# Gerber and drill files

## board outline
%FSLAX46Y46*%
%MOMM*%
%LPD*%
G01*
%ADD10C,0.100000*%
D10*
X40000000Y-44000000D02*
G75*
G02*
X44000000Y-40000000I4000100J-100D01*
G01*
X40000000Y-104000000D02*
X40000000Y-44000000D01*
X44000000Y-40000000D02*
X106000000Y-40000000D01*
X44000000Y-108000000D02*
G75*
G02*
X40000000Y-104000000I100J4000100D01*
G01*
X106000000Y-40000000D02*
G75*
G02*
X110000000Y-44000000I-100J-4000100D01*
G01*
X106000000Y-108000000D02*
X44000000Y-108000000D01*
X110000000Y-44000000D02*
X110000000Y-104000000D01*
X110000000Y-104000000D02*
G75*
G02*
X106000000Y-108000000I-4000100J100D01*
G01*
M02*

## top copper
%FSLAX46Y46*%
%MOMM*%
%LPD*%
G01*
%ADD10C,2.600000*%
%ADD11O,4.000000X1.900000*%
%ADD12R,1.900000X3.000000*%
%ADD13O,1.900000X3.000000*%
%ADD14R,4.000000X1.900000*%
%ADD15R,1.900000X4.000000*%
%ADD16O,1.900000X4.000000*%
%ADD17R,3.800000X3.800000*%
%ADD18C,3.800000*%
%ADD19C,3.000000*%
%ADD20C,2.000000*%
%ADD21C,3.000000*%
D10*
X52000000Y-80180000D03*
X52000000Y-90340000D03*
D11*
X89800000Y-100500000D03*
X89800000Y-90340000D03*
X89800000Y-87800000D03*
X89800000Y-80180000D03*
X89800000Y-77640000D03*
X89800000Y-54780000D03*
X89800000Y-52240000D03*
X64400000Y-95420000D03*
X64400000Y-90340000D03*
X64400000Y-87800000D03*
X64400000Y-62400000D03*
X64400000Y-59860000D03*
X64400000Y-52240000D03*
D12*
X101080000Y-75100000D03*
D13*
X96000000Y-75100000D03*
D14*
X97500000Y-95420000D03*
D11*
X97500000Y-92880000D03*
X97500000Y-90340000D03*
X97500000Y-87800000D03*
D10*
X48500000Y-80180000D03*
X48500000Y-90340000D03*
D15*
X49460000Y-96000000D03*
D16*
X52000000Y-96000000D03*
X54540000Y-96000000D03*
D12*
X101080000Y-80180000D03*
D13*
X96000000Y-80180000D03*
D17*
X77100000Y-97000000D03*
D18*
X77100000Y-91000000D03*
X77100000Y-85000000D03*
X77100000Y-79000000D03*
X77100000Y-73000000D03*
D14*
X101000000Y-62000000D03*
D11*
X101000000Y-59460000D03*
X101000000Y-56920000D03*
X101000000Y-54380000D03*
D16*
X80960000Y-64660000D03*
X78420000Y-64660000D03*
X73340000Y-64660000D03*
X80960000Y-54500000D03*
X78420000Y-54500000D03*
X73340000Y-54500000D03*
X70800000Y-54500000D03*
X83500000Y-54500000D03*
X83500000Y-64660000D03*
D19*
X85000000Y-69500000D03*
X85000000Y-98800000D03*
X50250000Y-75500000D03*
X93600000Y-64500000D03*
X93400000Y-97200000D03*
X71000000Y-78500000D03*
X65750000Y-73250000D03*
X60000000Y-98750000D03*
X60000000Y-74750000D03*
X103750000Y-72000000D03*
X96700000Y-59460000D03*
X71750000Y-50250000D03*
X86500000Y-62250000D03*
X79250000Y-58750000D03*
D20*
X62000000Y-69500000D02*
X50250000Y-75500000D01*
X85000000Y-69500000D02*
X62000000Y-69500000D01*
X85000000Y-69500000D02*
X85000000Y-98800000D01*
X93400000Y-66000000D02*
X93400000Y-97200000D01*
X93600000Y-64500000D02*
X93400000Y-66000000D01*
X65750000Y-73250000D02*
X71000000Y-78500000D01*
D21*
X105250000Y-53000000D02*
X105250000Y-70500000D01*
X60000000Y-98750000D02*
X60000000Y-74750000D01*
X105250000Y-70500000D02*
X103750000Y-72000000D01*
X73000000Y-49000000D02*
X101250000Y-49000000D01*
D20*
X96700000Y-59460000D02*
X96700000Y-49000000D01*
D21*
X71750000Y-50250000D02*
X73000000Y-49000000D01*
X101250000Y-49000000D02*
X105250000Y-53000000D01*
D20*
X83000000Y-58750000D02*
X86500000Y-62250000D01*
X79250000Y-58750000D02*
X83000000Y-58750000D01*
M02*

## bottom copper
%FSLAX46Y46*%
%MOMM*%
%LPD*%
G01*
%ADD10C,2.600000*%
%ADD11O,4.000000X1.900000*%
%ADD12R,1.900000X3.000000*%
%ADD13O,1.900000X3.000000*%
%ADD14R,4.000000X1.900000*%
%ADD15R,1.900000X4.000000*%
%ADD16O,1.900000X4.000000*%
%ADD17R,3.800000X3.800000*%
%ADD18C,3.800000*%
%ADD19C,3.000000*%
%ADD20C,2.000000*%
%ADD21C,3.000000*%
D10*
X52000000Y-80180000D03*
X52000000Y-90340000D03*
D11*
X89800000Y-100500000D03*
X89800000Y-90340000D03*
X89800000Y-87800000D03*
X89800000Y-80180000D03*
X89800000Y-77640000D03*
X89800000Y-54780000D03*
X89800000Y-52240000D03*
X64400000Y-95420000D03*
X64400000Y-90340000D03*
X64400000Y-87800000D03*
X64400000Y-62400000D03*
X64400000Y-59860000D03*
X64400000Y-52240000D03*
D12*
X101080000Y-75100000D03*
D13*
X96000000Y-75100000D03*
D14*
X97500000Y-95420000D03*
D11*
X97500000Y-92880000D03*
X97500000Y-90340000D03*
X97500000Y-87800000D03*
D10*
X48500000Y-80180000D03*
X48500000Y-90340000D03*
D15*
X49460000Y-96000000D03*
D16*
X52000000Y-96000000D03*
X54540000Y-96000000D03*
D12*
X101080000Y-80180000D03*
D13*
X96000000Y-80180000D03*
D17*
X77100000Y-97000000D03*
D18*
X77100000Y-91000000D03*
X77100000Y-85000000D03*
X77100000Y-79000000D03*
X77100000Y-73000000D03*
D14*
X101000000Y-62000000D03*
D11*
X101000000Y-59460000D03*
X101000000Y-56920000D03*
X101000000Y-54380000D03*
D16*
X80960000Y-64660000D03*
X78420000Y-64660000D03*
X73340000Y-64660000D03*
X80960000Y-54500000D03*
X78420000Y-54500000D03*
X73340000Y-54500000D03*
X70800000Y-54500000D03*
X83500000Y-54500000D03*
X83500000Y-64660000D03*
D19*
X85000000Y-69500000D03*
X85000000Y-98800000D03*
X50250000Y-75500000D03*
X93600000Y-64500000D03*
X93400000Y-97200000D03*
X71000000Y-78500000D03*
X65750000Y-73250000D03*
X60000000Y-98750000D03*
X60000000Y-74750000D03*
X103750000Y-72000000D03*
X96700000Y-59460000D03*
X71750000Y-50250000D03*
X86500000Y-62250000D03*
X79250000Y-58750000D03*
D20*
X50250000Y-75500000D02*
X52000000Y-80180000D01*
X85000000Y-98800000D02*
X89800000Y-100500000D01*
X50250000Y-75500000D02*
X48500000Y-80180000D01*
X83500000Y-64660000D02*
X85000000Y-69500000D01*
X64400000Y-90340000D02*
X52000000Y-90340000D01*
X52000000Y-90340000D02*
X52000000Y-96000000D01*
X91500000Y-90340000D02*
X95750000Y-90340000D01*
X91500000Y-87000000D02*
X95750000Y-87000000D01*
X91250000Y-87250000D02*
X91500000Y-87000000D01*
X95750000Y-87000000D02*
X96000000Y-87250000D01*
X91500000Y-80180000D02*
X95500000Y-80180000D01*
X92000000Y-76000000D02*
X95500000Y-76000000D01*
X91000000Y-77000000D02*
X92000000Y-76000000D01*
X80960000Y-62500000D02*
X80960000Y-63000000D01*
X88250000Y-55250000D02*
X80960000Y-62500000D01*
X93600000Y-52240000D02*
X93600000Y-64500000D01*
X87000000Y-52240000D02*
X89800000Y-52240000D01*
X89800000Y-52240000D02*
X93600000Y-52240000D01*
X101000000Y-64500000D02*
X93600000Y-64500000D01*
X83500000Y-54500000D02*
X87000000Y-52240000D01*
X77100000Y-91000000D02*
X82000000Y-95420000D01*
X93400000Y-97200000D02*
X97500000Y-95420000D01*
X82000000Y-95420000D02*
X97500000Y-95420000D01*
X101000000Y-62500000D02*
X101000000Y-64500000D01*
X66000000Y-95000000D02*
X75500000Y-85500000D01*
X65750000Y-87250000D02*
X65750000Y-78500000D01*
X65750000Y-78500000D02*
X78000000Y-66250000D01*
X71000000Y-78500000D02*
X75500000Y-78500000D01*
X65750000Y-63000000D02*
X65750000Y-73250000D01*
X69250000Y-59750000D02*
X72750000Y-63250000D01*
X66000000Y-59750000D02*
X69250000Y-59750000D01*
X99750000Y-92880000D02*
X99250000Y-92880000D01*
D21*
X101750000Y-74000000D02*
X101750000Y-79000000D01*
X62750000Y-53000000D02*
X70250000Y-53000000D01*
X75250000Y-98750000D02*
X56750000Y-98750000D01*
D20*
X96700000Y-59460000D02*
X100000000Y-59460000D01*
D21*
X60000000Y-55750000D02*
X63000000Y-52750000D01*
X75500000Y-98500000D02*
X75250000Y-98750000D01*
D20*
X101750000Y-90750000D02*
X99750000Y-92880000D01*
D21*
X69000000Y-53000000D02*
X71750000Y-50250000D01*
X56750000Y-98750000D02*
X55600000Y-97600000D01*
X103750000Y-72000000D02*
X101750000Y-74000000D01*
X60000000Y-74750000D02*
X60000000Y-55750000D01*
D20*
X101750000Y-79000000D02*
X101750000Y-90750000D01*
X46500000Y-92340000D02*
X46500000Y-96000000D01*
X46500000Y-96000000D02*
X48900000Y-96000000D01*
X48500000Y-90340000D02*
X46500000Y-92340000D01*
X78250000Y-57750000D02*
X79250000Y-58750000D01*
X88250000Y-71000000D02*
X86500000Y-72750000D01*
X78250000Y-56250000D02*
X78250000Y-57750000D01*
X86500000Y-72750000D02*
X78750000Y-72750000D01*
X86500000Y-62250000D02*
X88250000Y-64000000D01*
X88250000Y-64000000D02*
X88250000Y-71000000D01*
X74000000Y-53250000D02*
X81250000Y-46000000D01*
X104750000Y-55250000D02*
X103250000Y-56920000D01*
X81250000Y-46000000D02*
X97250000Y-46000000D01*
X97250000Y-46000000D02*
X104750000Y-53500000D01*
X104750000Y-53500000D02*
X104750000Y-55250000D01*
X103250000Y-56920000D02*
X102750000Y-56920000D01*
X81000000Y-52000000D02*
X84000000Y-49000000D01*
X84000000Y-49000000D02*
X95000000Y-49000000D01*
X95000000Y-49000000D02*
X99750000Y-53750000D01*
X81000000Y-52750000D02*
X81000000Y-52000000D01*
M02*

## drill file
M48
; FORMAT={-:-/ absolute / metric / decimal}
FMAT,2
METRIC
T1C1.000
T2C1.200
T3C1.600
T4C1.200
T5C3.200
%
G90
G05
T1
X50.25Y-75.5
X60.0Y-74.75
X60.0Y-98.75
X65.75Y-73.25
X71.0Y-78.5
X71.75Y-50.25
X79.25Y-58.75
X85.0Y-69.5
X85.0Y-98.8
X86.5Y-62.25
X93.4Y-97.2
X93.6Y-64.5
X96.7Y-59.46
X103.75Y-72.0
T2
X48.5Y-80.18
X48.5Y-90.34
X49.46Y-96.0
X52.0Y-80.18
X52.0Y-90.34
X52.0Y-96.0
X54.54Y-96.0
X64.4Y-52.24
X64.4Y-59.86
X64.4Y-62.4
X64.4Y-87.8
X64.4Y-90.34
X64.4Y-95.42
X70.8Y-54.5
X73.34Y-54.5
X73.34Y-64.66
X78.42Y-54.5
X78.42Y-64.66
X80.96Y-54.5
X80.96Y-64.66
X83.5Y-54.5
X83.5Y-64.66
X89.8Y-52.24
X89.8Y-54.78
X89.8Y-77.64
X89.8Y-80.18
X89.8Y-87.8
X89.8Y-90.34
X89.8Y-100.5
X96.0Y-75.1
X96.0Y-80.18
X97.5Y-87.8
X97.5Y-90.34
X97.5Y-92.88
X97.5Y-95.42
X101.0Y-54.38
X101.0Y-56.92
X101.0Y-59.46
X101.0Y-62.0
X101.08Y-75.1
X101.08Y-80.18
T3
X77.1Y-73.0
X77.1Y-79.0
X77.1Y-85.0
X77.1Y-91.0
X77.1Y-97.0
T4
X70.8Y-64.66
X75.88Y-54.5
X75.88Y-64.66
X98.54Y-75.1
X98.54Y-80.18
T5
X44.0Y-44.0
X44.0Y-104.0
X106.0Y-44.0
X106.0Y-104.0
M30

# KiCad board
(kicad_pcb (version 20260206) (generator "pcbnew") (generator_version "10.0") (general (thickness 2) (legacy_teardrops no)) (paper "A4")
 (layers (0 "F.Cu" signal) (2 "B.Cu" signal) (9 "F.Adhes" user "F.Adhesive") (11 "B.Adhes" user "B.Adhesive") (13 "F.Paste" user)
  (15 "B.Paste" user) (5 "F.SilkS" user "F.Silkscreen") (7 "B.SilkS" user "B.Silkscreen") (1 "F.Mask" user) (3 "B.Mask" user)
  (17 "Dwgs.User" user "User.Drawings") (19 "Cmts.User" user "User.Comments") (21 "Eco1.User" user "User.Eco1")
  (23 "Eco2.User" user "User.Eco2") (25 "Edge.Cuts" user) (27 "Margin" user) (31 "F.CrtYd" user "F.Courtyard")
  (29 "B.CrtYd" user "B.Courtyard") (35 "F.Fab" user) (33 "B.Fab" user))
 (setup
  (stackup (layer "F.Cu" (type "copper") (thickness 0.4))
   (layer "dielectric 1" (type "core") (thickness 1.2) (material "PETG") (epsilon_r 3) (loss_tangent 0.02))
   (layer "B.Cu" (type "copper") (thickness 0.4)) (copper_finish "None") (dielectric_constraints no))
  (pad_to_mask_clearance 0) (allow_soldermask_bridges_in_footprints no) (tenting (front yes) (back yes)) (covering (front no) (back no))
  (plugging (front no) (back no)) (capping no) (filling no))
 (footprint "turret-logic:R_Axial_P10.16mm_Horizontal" (layer "F.Cu") (at 52 80.18 -90)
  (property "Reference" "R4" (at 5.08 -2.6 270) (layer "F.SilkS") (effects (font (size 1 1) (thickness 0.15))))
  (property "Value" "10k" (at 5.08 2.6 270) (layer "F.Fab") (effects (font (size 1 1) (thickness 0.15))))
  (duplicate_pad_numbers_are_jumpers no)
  (pad "1" thru_hole circle (at 0 0 270) (size 2.6 2.6) (drill 1.2) (layers "*.Cu" "*.Mask") (remove_unused_layers no) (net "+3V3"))
  (pad "2" thru_hole circle (at 10.16 0 270) (size 2.6 2.6) (drill 1.2) (layers "*.Cu" "*.Mask") (remove_unused_layers no) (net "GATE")))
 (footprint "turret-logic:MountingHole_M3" (layer "F.Cu") (at 106 44)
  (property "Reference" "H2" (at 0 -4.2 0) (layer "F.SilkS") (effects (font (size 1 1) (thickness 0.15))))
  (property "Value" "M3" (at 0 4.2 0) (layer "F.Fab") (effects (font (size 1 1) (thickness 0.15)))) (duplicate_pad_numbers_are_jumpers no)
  (pad "" np_thru_hole circle (at 0 0) (size 3.2 3.2) (drill 3.2) (layers "*.Cu" "*.Mask")))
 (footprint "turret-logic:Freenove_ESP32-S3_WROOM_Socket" (layer "F.Cu") (at 89.8 100.5 90)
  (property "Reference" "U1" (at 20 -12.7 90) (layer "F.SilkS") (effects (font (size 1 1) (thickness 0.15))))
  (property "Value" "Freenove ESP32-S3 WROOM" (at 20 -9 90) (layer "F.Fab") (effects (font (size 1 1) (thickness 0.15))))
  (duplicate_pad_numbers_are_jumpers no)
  (pad "L1" thru_hole oval (at 0 0 90) (size 1.9 4) (drill 1.2) (layers "*.Cu" "B.Mask") (remove_unused_layers no) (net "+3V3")
   (zone_connect 0))
  (pad "L5" thru_hole oval (at 10.16 0 90) (size 1.9 4) (drill 1.2) (layers "*.Cu" "B.Mask") (remove_unused_layers no) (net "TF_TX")
   (zone_connect 0))
  (pad "L6" thru_hole oval (at 12.7 0 90) (size 1.9 4) (drill 1.2) (layers "*.Cu" "B.Mask") (remove_unused_layers no) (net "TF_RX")
   (zone_connect 0))
  (pad "L9" thru_hole oval (at 20.32 0 90) (size 1.9 4) (drill 1.2) (layers "*.Cu" "B.Mask") (remove_unused_layers no) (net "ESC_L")
   (zone_connect 0))
  (pad "L10" thru_hole oval (at 22.86 0 90) (size 1.9 4) (drill 1.2) (layers "*.Cu" "B.Mask") (remove_unused_layers no) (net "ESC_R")
   (zone_connect 0))
  (pad "L19" thru_hole oval (at 45.72 0 90) (size 1.9 4) (drill 1.2) (layers "*.Cu" "B.Mask") (remove_unused_layers no) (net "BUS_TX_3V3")
   (zone_connect 0))
  (pad "L20" thru_hole oval (at 48.26 0 90) (size 1.9 4) (drill 1.2) (layers "*.Cu" "B.Mask") (remove_unused_layers no) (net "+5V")
   (zone_connect 0))
  (pad "R3" thru_hole oval (at 5.08 -25.4 90) (size 1.9 4) (drill 1.2) (layers "*.Cu" "B.Mask") (remove_unused_layers no) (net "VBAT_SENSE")
   (zone_connect 0))
  (pad "R5" thru_hole oval (at 10.16 -25.4 90) (size 1.9 4) (drill 1.2) (layers "*.Cu" "B.Mask") (remove_unused_layers no) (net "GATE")
   (zone_connect 0))
  (pad "R6" thru_hole oval (at 12.7 -25.4 90) (size 1.9 4) (drill 1.2) (layers "*.Cu" "B.Mask") (remove_unused_layers no)
   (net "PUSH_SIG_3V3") (zone_connect 0))
  (pad "R16" thru_hole oval (at 38.1 -25.4 90) (size 1.9 4) (drill 1.2) (layers "*.Cu" "B.Mask") (remove_unused_layers no) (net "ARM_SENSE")
   (zone_connect 0))
  (pad "R17" thru_hole oval (at 40.64 -25.4 90) (size 1.9 4) (drill 1.2) (layers "*.Cu" "B.Mask") (remove_unused_layers no)
   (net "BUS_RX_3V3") (zone_connect 0))
  (pad "R20" thru_hole oval (at 48.26 -25.4 90) (size 1.9 4) (drill 1.2) (layers "*.Cu" "B.Mask") (remove_unused_layers no) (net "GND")
   (zone_connect 0)))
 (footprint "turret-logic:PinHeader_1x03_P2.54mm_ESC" (layer "F.Cu") (at 101.08 75.1 180)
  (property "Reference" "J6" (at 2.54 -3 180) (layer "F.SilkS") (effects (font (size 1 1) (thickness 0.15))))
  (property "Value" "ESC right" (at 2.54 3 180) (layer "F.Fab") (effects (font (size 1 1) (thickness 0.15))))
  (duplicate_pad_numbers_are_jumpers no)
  (pad "" np_thru_hole circle (at 2.54 0) (size 1.2 1.2) (drill 1.2) (layers "*.Cu" "*.Mask"))
  (pad "1" thru_hole rect (at 0 0 180) (size 1.9 3) (drill 1.2) (layers "*.Cu" "B.Mask") (remove_unused_layers no) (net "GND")
   (zone_connect 0))
  (pad "3" thru_hole oval (at 5.08 0 180) (size 1.9 3) (drill 1.2) (layers "*.Cu" "B.Mask") (remove_unused_layers no) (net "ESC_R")
   (zone_connect 0)))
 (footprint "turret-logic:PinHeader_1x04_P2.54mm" (layer "F.Cu") (at 97.5 95.42 90)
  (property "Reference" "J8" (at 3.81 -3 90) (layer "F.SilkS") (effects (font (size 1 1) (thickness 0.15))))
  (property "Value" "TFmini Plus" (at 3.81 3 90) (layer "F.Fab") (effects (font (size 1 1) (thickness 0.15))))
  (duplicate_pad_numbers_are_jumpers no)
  (pad "1" thru_hole rect (at 0 0 90) (size 1.9 4) (drill 1.2) (layers "*.Cu" "B.Mask") (remove_unused_layers no) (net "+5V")
   (zone_connect 0))
  (pad "2" thru_hole oval (at 2.54 0 90) (size 1.9 4) (drill 1.2) (layers "*.Cu" "B.Mask") (remove_unused_layers no) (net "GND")
   (zone_connect 0))
  (pad "3" thru_hole oval (at 5.08 0 90) (size 1.9 4) (drill 1.2) (layers "*.Cu" "B.Mask") (remove_unused_layers no) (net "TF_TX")
   (zone_connect 0))
  (pad "4" thru_hole oval (at 7.62 0 90) (size 1.9 4) (drill 1.2) (layers "*.Cu" "B.Mask") (remove_unused_layers no) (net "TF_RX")
   (zone_connect 0)))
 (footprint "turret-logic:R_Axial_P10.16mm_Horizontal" (layer "F.Cu") (at 48.5 80.18 -90)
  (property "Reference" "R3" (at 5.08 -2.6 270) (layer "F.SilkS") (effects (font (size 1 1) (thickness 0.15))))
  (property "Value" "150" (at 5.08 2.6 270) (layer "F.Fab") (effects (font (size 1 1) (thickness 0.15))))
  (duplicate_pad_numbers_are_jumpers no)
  (pad "1" thru_hole circle (at 0 0 270) (size 2.6 2.6) (drill 1.2) (layers "*.Cu" "*.Mask") (remove_unused_layers no) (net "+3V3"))
  (pad "2" thru_hole circle (at 10.16 0 270) (size 2.6 2.6) (drill 1.2) (layers "*.Cu" "*.Mask") (remove_unused_layers no) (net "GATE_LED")))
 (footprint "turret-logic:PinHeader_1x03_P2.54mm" (layer "F.Cu") (at 49.46 96)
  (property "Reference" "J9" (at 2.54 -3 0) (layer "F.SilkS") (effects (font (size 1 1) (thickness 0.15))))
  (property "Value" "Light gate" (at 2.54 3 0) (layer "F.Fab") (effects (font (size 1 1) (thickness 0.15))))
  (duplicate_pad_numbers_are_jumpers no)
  (pad "1" thru_hole rect (at 0 0) (size 1.9 4) (drill 1.2) (layers "*.Cu" "B.Mask") (remove_unused_layers no) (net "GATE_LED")
   (zone_connect 0))
  (pad "2" thru_hole oval (at 2.54 0) (size 1.9 4) (drill 1.2) (layers "*.Cu" "B.Mask") (remove_unused_layers no) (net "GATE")
   (zone_connect 0))
  (pad "3" thru_hole oval (at 5.08 0) (size 1.9 4) (drill 1.2) (layers "*.Cu" "B.Mask") (remove_unused_layers no) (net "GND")
   (zone_connect 0)))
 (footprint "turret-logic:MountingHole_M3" (layer "F.Cu") (at 44 44)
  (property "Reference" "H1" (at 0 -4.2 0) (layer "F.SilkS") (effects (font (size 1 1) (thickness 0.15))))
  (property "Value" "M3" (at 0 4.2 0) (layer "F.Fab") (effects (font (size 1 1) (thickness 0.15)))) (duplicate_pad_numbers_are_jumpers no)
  (pad "" np_thru_hole circle (at 0 0) (size 3.2 3.2) (drill 3.2) (layers "*.Cu" "*.Mask")))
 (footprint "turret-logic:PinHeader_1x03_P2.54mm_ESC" (layer "F.Cu") (at 101.08 80.18 180)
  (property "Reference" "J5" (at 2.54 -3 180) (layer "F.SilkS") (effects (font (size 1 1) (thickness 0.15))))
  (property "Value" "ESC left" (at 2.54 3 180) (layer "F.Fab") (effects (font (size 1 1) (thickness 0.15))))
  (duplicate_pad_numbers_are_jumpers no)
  (pad "" np_thru_hole circle (at 2.54 0) (size 1.2 1.2) (drill 1.2) (layers "*.Cu" "*.Mask"))
  (pad "1" thru_hole rect (at 0 0 180) (size 1.9 3) (drill 1.2) (layers "*.Cu" "B.Mask") (remove_unused_layers no) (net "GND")
   (zone_connect 0))
  (pad "3" thru_hole oval (at 5.08 0 180) (size 1.9 3) (drill 1.2) (layers "*.Cu" "B.Mask") (remove_unused_layers no) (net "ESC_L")
   (zone_connect 0)))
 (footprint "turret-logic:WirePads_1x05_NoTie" (layer "F.Cu") (at 77.1 97 90)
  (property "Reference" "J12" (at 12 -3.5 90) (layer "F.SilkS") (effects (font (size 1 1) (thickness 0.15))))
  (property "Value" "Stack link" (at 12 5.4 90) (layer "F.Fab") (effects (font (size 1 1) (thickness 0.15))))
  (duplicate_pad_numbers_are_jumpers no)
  (pad "1" thru_hole rect (at 0 0 90) (size 3.8 3.8) (drill 1.6) (layers "*.Cu" "*.Mask") (remove_unused_layers no) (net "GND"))
  (pad "2" thru_hole circle (at 6 0 90) (size 3.8 3.8) (drill 1.6) (layers "*.Cu" "*.Mask") (remove_unused_layers no) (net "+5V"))
  (pad "3" thru_hole circle (at 12 0 90) (size 3.8 3.8) (drill 1.6) (layers "*.Cu" "*.Mask") (remove_unused_layers no) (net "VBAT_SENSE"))
  (pad "4" thru_hole circle (at 18 0 90) (size 3.8 3.8) (drill 1.6) (layers "*.Cu" "*.Mask") (remove_unused_layers no) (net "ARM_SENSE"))
  (pad "5" thru_hole circle (at 24 0 90) (size 3.8 3.8) (drill 1.6) (layers "*.Cu" "*.Mask") (remove_unused_layers no) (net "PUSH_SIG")))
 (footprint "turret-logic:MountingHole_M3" (layer "F.Cu") (at 44 104)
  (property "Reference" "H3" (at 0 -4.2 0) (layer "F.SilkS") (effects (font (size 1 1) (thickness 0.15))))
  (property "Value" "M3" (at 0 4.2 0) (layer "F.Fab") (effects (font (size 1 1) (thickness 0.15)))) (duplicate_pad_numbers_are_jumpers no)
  (pad "" np_thru_hole circle (at 0 0) (size 3.2 3.2) (drill 3.2) (layers "*.Cu" "*.Mask")))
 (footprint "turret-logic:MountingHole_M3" (layer "F.Cu") (at 106 104)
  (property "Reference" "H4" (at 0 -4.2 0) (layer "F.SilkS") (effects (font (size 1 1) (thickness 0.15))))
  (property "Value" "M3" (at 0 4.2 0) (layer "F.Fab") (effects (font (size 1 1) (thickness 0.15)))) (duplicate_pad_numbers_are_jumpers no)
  (pad "" np_thru_hole circle (at 0 0) (size 3.2 3.2) (drill 3.2) (layers "*.Cu" "*.Mask")))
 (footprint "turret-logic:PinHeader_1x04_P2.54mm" (layer "F.Cu") (at 101 62 90)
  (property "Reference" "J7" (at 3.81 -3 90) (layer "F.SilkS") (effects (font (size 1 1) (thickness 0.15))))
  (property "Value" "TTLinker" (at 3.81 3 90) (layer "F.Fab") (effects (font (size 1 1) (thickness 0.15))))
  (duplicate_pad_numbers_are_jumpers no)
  (pad "1" thru_hole rect (at 0 0 90) (size 1.9 4) (drill 1.2) (layers "*.Cu" "B.Mask") (remove_unused_layers no) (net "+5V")
   (zone_connect 0))
  (pad "2" thru_hole oval (at 2.54 0 90) (size 1.9 4) (drill 1.2) (layers "*.Cu" "B.Mask") (remove_unused_layers no) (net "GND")
   (zone_connect 0))
  (pad "3" thru_hole oval (at 5.08 0 90) (size 1.9 4) (drill 1.2) (layers "*.Cu" "B.Mask") (remove_unused_layers no) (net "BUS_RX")
   (zone_connect 0))
  (pad "4" thru_hole oval (at 7.62 0 90) (size 1.9 4) (drill 1.2) (layers "*.Cu" "B.Mask") (remove_unused_layers no) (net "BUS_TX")
   (zone_connect 0)))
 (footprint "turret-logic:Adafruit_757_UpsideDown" (layer "F.Cu") (at 83.5 64.66 180)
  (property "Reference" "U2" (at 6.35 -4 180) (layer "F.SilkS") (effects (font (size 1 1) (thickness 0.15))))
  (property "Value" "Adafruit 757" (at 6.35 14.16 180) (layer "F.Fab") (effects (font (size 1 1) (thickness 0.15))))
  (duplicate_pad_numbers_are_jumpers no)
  (pad "" np_thru_hole circle (at 7.62 0) (size 1.2 1.2) (drill 1.2) (layers "*.Cu" "*.Mask"))
  (pad "" np_thru_hole circle (at 7.62 10.16) (size 1.2 1.2) (drill 1.2) (layers "*.Cu" "*.Mask"))
  (pad "" np_thru_hole circle (at 12.7 0) (size 1.2 1.2) (drill 1.2) (layers "*.Cu" "*.Mask"))
  (pad "A1" thru_hole oval (at 2.54 0 180) (size 1.9 4) (drill 1.2) (layers "*.Cu" "B.Mask") (remove_unused_layers no) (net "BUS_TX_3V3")
   (zone_connect 0))
  (pad "A2" thru_hole oval (at 5.08 0 180) (size 1.9 4) (drill 1.2) (layers "*.Cu" "B.Mask") (remove_unused_layers no) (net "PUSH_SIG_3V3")
   (zone_connect 0))
  (pad "A4" thru_hole oval (at 10.16 0 180) (size 1.9 4) (drill 1.2) (layers "*.Cu" "B.Mask") (remove_unused_layers no) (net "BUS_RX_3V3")
   (zone_connect 0))
  (pad "B1" thru_hole oval (at 2.54 10.16 180) (size 1.9 4) (drill 1.2) (layers "*.Cu" "B.Mask") (remove_unused_layers no) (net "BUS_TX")
   (zone_connect 0))
  (pad "B2" thru_hole oval (at 5.08 10.16 180) (size 1.9 4) (drill 1.2) (layers "*.Cu" "B.Mask") (remove_unused_layers no) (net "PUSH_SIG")
   (zone_connect 0))
  (pad "B4" thru_hole oval (at 10.16 10.16 180) (size 1.9 4) (drill 1.2) (layers "*.Cu" "B.Mask") (remove_unused_layers no) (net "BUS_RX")
   (zone_connect 0))
  (pad "GND" thru_hole oval (at 12.7 10.16 180) (size 1.9 4) (drill 1.2) (layers "*.Cu" "B.Mask") (remove_unused_layers no) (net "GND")
   (zone_connect 0))
  (pad "HV" thru_hole oval (at 0 10.16 180) (size 1.9 4) (drill 1.2) (layers "*.Cu" "B.Mask") (remove_unused_layers no) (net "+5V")
   (zone_connect 0))
  (pad "LV" thru_hole oval (at 0 0 180) (size 1.9 4) (drill 1.2) (layers "*.Cu" "B.Mask") (remove_unused_layers no) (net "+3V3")
   (zone_connect 0)))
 (gr_arc (start 40 44) (mid 41.1716 41.1716) (end 44 40) (stroke (width 0.1) (type default)) (layer "Edge.Cuts"))
 (gr_line (start 40 104) (end 40 44) (stroke (width 0.1) (type default)) (layer "Edge.Cuts"))
 (gr_line (start 44 40) (end 106 40) (stroke (width 0.1) (type default)) (layer "Edge.Cuts"))
 (gr_arc (start 44 108) (mid 41.1716 106.8284) (end 40 104) (stroke (width 0.1) (type default)) (layer "Edge.Cuts"))
 (gr_arc (start 106 40) (mid 108.8284 41.1716) (end 110 44) (stroke (width 0.1) (type default)) (layer "Edge.Cuts"))
 (gr_line (start 106 108) (end 44 108) (stroke (width 0.1) (type default)) (layer "Edge.Cuts"))
 (gr_line (start 110 44) (end 110 104) (stroke (width 0.1) (type default)) (layer "Edge.Cuts"))
 (gr_arc (start 110 104) (mid 108.8284 106.8284) (end 106 108) (stroke (width 0.1) (type default)) (layer "Edge.Cuts"))
 (segment (start 62 69.5) (end 50.25 75.5) (width 2) (layer "F.Cu") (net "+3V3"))
 (segment (start 85 69.5) (end 62 69.5) (width 2) (layer "F.Cu") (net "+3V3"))
 (segment (start 85 69.5) (end 85 98.8) (width 2) (layer "F.Cu") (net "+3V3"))
 (via (at 85 69.5) (size 3) (drill 1) (layers "F.Cu" "B.Cu") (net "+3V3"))
 (via (at 85 98.8) (size 3) (drill 1) (layers "F.Cu" "B.Cu") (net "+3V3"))
 (via (at 50.25 75.5) (size 3) (drill 1) (layers "F.Cu" "B.Cu") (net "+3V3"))
 (segment (start 50.25 75.5) (end 52 80.18) (width 2) (layer "B.Cu") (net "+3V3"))
 (segment (start 85 98.8) (end 89.8 100.5) (width 2) (layer "B.Cu") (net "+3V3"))
 (segment (start 50.25 75.5) (end 48.5 80.18) (width 2) (layer "B.Cu") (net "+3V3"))
 (segment (start 83.5 64.66) (end 85 69.5) (width 2) (layer "B.Cu") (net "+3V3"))
 (segment (start 64.4 90.34) (end 52 90.34) (width 2) (layer "B.Cu") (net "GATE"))
 (segment (start 52 90.34) (end 52 96) (width 2) (layer "B.Cu") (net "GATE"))
 (segment (start 91.5 90.34) (end 95.75 90.34) (width 2) (layer "B.Cu") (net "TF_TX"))
 (segment (start 91.5 87) (end 95.75 87) (width 2) (layer "B.Cu") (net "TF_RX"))
 (segment (start 91.25 87.25) (end 91.5 87) (width 2) (layer "B.Cu") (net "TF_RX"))
 (segment (start 95.75 87) (end 96 87.25) (width 2) (layer "B.Cu") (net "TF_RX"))
 (segment (start 91.5 80.18) (end 95.5 80.18) (width 2) (layer "B.Cu") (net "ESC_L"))
 (segment (start 92 76) (end 95.5 76) (width 2) (layer "B.Cu") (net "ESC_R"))
 (segment (start 91 77) (end 92 76) (width 2) (layer "B.Cu") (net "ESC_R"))
 (segment (start 80.96 62.5) (end 80.96 63) (width 2) (layer "B.Cu") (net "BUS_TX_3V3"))
 (segment (start 88.25 55.25) (end 80.96 62.5) (width 2) (layer "B.Cu") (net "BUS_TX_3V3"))
 (segment (start 93.4 66) (end 93.4 97.2) (width 2) (layer "F.Cu") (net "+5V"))
 (segment (start 93.6 64.5) (end 93.4 66) (width 2) (layer "F.Cu") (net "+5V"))
 (via (at 93.6 64.5) (size 3) (drill 1) (layers "F.Cu" "B.Cu") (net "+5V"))
 (via (at 93.4 97.2) (size 3) (drill 1) (layers "F.Cu" "B.Cu") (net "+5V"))
 (segment (start 93.6 52.24) (end 93.6 64.5) (width 2) (layer "B.Cu") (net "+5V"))
 (segment (start 87 52.24) (end 89.8 52.24) (width 2) (layer "B.Cu") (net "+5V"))
 (segment (start 89.8 52.24) (end 93.6 52.24) (width 2) (layer "B.Cu") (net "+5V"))
 (segment (start 101 64.5) (end 93.6 64.5) (width 2) (layer "B.Cu") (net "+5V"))
 (segment (start 83.5 54.5) (end 87 52.24) (width 2) (layer "B.Cu") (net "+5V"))
 (segment (start 77.1 91) (end 82 95.42) (width 2) (layer "B.Cu") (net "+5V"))
 (segment (start 93.4 97.2) (end 97.5 95.42) (width 2) (layer "B.Cu") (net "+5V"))
 (segment (start 82 95.42) (end 97.5 95.42) (width 2) (layer "B.Cu") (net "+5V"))
 (segment (start 101 62.5) (end 101 64.5) (width 2) (layer "B.Cu") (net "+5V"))
 (segment (start 66 95) (end 75.5 85.5) (width 2) (layer "B.Cu") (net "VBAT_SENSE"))
 (segment (start 65.75 87.25) (end 65.75 78.5) (width 2) (layer "B.Cu") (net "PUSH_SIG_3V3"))
 (segment (start 65.75 78.5) (end 78 66.25) (width 2) (layer "B.Cu") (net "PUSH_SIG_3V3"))
 (segment (start 65.75 73.25) (end 71 78.5) (width 2) (layer "F.Cu") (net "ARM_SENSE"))
 (via (at 71 78.5) (size 3) (drill 1) (layers "F.Cu" "B.Cu") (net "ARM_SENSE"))
 (via (at 65.75 73.25) (size 3) (drill 1) (layers "F.Cu" "B.Cu") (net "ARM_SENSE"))
 (segment (start 71 78.5) (end 75.5 78.5) (width 2) (layer "B.Cu") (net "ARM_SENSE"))
 (segment (start 65.75 63) (end 65.75 73.25) (width 2) (layer "B.Cu") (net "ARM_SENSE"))
 (segment (start 69.25 59.75) (end 72.75 63.25) (width 2) (layer "B.Cu") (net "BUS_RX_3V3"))
 (segment (start 66 59.75) (end 69.25 59.75) (width 2) (layer "B.Cu") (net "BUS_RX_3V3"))
 (segment (start 105.25 53) (end 105.25 70.5) (width 3) (layer "F.Cu") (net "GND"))
 (segment (start 60 98.75) (end 60 74.75) (width 3) (layer "F.Cu") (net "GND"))
 (segment (start 105.25 70.5) (end 103.75 72) (width 3) (layer "F.Cu") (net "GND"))
 (segment (start 73 49) (end 101.25 49) (width 3) (layer "F.Cu") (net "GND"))
 (segment (start 96.7 59.46) (end 96.7 49) (width 2) (layer "F.Cu") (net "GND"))
 (segment (start 71.75 50.25) (end 73 49) (width 3) (layer "F.Cu") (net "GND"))
 (segment (start 101.25 49) (end 105.25 53) (width 3) (layer "F.Cu") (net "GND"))
 (via (at 60 98.75) (size 3) (drill 1) (layers "F.Cu" "B.Cu") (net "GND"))
 (via (at 60 74.75) (size 3) (drill 1) (layers "F.Cu" "B.Cu") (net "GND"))
 (via (at 103.75 72) (size 3) (drill 1) (layers "F.Cu" "B.Cu") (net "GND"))
 (via (at 96.7 59.46) (size 3) (drill 1) (layers "F.Cu" "B.Cu") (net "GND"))
 (via (at 71.75 50.25) (size 3) (drill 1) (layers "F.Cu" "B.Cu") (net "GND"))
 (segment (start 99.75 92.88) (end 99.25 92.88) (width 2) (layer "B.Cu") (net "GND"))
 (segment (start 101.75 74) (end 101.75 79) (width 3) (layer "B.Cu") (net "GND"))
 (segment (start 62.75 53) (end 70.25 53) (width 3) (layer "B.Cu") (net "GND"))
 (segment (start 75.25 98.75) (end 56.75 98.75) (width 3) (layer "B.Cu") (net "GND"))
 (segment (start 96.7 59.46) (end 100 59.46) (width 2) (layer "B.Cu") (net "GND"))
 (segment (start 60 55.75) (end 63 52.75) (width 3) (layer "B.Cu") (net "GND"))
 (segment (start 75.5 98.5) (end 75.25 98.75) (width 3) (layer "B.Cu") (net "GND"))
 (segment (start 101.75 90.75) (end 99.75 92.88) (width 2) (layer "B.Cu") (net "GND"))
 (segment (start 69 53) (end 71.75 50.25) (width 3) (layer "B.Cu") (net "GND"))
 (segment (start 56.75 98.75) (end 55.6 97.6) (width 3) (layer "B.Cu") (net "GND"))
 (segment (start 103.75 72) (end 101.75 74) (width 3) (layer "B.Cu") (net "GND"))
 (segment (start 60 74.75) (end 60 55.75) (width 3) (layer "B.Cu") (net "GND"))
 (segment (start 101.75 79) (end 101.75 90.75) (width 2) (layer "B.Cu") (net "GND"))
 (segment (start 46.5 92.34) (end 46.5 96) (width 2) (layer "B.Cu") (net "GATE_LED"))
 (segment (start 46.5 96) (end 48.9 96) (width 2) (layer "B.Cu") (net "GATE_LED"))
 (segment (start 48.5 90.34) (end 46.5 92.34) (width 2) (layer "B.Cu") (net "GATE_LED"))
 (segment (start 83 58.75) (end 86.5 62.25) (width 2) (layer "F.Cu") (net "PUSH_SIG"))
 (segment (start 79.25 58.75) (end 83 58.75) (width 2) (layer "F.Cu") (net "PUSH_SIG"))
 (via (at 86.5 62.25) (size 3) (drill 1) (layers "F.Cu" "B.Cu") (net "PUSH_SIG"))
 (via (at 79.25 58.75) (size 3) (drill 1) (layers "F.Cu" "B.Cu") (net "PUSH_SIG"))
 (segment (start 78.25 57.75) (end 79.25 58.75) (width 2) (layer "B.Cu") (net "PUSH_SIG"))
 (segment (start 88.25 71) (end 86.5 72.75) (width 2) (layer "B.Cu") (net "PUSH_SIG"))
 (segment (start 78.25 56.25) (end 78.25 57.75) (width 2) (layer "B.Cu") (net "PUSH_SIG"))
 (segment (start 86.5 72.75) (end 78.75 72.75) (width 2) (layer "B.Cu") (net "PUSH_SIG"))
 (segment (start 86.5 62.25) (end 88.25 64) (width 2) (layer "B.Cu") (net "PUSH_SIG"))
 (segment (start 88.25 64) (end 88.25 71) (width 2) (layer "B.Cu") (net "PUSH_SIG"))
 (segment (start 74 53.25) (end 81.25 46) (width 2) (layer "B.Cu") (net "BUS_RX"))
 (segment (start 104.75 55.25) (end 103.25 56.92) (width 2) (layer "B.Cu") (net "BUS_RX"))
 (segment (start 81.25 46) (end 97.25 46) (width 2) (layer "B.Cu") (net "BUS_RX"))
 (segment (start 97.25 46) (end 104.75 53.5) (width 2) (layer "B.Cu") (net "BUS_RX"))
 (segment (start 104.75 53.5) (end 104.75 55.25) (width 2) (layer "B.Cu") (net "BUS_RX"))
 (segment (start 103.25 56.92) (end 102.75 56.92) (width 2) (layer "B.Cu") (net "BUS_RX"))
 (segment (start 81 52) (end 84 49) (width 2) (layer "B.Cu") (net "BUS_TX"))
 (segment (start 84 49) (end 95 49) (width 2) (layer "B.Cu") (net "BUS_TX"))
 (segment (start 95 49) (end 99.75 53.75) (width 2) (layer "B.Cu") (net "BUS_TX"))
 (segment (start 81 52.75) (end 81 52) (width 2) (layer "B.Cu") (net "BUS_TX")))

